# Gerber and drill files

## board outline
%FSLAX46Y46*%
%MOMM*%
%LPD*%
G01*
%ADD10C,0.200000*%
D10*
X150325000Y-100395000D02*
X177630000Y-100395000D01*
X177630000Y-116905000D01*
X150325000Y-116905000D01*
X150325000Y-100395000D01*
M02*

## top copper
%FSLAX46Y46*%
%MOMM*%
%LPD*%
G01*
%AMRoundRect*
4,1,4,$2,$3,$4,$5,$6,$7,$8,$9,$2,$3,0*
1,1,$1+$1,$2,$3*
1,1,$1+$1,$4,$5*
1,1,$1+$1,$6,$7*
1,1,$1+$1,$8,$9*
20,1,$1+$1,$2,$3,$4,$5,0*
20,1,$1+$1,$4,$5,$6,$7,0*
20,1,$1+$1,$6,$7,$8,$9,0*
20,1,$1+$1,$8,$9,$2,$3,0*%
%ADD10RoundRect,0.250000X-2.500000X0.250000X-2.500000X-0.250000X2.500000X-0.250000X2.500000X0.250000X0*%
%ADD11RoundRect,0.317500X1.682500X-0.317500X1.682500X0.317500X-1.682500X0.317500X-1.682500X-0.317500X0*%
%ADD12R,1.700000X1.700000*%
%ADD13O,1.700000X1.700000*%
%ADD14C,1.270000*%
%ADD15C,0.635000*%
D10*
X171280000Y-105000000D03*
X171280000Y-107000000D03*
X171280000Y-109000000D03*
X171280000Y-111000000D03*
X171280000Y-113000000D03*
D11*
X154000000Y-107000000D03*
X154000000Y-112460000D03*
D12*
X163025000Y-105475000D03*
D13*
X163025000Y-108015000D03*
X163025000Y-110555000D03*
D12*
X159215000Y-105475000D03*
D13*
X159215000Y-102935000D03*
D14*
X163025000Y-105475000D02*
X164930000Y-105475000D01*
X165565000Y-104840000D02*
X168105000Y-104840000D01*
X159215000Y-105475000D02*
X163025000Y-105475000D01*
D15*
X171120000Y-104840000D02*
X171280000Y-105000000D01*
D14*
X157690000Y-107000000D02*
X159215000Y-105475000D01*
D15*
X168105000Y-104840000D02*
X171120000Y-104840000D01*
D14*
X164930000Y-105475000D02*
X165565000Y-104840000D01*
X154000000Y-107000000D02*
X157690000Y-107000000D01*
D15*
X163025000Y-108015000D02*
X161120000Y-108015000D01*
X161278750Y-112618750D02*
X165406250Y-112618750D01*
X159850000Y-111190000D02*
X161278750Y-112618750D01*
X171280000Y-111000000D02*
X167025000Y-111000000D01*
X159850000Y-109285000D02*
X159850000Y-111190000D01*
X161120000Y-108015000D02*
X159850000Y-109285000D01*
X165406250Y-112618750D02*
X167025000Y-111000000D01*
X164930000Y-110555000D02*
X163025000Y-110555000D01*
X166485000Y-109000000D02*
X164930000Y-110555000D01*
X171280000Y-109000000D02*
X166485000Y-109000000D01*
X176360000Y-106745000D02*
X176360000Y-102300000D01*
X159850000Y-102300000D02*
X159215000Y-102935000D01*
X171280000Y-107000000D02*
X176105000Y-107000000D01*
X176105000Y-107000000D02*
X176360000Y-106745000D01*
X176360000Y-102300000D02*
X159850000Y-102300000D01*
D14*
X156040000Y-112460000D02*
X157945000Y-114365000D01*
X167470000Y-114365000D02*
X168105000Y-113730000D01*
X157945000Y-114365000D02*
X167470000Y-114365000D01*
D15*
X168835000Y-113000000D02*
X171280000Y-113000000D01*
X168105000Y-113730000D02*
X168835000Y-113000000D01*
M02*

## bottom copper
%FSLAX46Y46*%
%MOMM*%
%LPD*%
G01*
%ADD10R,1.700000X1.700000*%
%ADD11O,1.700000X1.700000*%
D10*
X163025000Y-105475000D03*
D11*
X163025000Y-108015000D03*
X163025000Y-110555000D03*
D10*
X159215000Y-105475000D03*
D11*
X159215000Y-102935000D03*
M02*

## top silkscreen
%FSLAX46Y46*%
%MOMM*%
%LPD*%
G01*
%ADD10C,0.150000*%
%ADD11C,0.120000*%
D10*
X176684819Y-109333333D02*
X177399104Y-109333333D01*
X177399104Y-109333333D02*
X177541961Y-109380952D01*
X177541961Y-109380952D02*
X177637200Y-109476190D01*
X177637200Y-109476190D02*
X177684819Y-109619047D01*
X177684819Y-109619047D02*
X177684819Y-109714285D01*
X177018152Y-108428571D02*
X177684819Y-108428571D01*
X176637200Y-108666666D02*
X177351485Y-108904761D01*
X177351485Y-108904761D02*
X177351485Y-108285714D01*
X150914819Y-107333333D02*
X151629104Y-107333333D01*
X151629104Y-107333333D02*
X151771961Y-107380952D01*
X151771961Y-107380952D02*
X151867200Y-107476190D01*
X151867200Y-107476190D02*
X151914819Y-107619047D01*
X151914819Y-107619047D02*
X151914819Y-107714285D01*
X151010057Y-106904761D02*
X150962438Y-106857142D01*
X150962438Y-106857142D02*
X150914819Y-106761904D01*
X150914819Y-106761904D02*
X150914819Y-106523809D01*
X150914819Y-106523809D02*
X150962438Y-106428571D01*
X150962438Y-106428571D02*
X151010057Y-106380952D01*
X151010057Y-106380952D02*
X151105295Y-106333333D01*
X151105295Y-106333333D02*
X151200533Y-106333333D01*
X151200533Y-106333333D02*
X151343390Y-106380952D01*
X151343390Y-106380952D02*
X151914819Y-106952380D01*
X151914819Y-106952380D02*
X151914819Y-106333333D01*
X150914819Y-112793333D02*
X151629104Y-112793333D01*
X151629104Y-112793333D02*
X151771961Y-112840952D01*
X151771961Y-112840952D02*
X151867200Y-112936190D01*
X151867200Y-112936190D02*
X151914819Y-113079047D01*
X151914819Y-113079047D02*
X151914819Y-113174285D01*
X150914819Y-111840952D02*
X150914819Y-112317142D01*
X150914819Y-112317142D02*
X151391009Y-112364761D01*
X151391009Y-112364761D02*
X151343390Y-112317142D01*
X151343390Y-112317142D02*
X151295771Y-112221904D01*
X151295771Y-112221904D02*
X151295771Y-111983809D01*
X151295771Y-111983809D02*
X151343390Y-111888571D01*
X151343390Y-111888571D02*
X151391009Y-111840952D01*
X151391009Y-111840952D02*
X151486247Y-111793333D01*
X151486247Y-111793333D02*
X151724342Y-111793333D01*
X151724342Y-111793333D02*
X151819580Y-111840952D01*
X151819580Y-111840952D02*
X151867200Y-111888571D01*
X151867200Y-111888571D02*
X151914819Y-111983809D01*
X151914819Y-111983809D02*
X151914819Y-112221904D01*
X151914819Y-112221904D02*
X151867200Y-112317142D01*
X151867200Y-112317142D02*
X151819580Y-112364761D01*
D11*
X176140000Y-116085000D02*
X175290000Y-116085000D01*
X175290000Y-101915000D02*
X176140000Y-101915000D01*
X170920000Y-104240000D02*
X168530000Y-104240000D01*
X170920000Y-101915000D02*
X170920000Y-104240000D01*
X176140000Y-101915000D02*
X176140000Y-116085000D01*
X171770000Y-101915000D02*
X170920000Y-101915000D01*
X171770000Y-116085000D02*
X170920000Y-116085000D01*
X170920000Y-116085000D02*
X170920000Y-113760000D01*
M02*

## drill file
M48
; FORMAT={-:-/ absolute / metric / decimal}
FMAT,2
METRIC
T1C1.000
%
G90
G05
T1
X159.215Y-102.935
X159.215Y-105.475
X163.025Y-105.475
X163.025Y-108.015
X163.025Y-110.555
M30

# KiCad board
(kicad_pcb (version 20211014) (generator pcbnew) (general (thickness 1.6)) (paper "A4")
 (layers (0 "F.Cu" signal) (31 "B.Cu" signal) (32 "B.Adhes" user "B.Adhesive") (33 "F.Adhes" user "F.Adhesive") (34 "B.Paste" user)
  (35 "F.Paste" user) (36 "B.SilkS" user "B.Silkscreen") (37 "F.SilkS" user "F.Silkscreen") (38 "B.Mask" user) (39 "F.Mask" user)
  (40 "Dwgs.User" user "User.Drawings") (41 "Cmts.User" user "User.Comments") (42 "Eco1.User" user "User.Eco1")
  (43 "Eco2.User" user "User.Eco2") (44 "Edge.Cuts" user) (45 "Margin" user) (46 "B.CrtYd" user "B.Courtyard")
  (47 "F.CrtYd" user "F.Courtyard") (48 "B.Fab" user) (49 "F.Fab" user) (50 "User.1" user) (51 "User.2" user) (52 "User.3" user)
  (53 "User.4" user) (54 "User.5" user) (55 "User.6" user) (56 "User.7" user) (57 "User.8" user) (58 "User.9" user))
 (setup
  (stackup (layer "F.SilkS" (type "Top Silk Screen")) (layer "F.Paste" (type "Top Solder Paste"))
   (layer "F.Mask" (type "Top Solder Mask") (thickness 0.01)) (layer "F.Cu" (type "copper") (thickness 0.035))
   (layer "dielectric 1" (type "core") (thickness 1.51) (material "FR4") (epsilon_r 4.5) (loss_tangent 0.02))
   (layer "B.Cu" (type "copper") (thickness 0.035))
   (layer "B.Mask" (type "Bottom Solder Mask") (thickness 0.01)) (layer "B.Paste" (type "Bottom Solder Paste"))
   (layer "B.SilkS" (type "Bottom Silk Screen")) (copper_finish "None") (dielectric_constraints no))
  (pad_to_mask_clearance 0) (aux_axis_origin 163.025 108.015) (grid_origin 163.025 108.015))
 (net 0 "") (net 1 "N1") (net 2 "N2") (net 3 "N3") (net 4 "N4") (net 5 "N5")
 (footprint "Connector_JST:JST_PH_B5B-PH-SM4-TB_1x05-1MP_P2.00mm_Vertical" (layer "F.Cu") (at 171.78 109 -90)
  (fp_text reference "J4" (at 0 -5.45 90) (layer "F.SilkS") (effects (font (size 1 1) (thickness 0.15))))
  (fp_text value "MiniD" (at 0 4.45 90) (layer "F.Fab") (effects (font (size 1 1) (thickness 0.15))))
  (fp_line (start 7.085 -4.36) (end 7.085 -3.51) (layer "F.SilkS") (width 0.12))
  (fp_line (start -7.085 -3.51) (end -7.085 -4.36) (layer "F.SilkS") (width 0.12))
  (fp_line (start -4.76 0.86) (end -4.76 3.25) (layer "F.SilkS") (width 0.12))
  (fp_line (start -7.085 0.86) (end -4.76 0.86) (layer "F.SilkS") (width 0.12))
  (fp_line (start -7.085 -4.36) (end 7.085 -4.36) (layer "F.SilkS") (width 0.12))
  (fp_line (start -7.085 0.01) (end -7.085 0.86) (layer "F.SilkS") (width 0.12))
  (fp_line (start 7.085 0.01) (end 7.085 0.86) (layer "F.SilkS") (width 0.12))
  (fp_line (start 7.085 0.86) (end 4.76 0.86) (layer "F.SilkS") (width 0.12))
  (pad "1" smd roundrect (at -4 0.5 270) (size 1 5.5) (layers "F.Cu" "F.Paste" "F.Mask") (roundrect_rratio 0.25) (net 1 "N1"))
  (pad "2" smd roundrect (at -2 0.5 270) (size 1 5.5) (layers "F.Cu" "F.Paste" "F.Mask") (roundrect_rratio 0.25) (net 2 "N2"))
  (pad "3" smd roundrect (at 0 0.5 270) (size 1 5.5) (layers "F.Cu" "F.Paste" "F.Mask") (roundrect_rratio 0.25) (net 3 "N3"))
  (pad "4" smd roundrect (at 2 0.5 270) (size 1 5.5) (layers "F.Cu" "F.Paste" "F.Mask") (roundrect_rratio 0.25) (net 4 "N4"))
  (pad "5" smd roundrect (at 4 0.5 270) (size 1 5.5) (layers "F.Cu" "F.Paste" "F.Mask") (roundrect_rratio 0.25) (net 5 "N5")))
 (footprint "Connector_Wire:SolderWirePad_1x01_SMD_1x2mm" (layer "F.Cu") (at 154 107 90)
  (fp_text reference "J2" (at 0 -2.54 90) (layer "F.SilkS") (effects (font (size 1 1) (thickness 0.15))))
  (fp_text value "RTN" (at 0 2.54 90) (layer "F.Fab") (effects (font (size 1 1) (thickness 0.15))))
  (pad "1" smd roundrect (at 0 0 90) (size 1.27 4) (layers "F.Cu" "F.Paste" "F.Mask") (roundrect_rratio 0.25) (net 1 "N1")))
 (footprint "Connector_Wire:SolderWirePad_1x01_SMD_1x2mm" (layer "F.Cu") (at 154 112.46 90)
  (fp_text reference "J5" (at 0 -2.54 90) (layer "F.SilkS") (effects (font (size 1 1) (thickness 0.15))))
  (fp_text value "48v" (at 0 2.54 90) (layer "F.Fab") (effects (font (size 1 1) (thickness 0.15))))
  (pad "1" smd roundrect (at 0 0 90) (size 1.27 4) (layers "F.Cu" "F.Paste" "F.Mask") (roundrect_rratio 0.25) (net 5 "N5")))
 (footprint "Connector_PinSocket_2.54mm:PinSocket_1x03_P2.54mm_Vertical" (layer "B.Cu") (at 163.025 105.475 180)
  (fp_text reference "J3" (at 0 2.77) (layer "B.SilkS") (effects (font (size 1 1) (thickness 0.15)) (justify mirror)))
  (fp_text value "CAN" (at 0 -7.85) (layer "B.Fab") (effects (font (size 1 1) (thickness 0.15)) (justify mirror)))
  (pad "1" thru_hole rect (at 0 0 180) (size 1.7 1.7) (drill 1) (layers *.Cu *.Mask) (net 1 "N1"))
  (pad "2" thru_hole oval (at 0 -2.54 180) (size 1.7 1.7) (drill 1) (layers *.Cu *.Mask) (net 4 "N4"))
  (pad "3" thru_hole oval (at 0 -5.08 180) (size 1.7 1.7) (drill 1) (layers *.Cu *.Mask) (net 3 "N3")))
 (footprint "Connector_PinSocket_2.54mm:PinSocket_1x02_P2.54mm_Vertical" (layer "B.Cu") (at 159.215 105.475)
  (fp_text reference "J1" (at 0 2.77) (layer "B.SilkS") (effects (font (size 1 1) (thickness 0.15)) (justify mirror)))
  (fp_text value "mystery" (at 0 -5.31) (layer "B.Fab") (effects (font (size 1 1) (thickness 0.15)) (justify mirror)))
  (pad "1" thru_hole rect (at 0 0) (size 1.7 1.7) (drill 1) (layers *.Cu *.Mask) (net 1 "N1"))
  (pad "2" thru_hole oval (at 0 -2.54) (size 1.7 1.7) (drill 1) (layers *.Cu *.Mask) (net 2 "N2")))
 (gr_rect (start 150.325 100.395) (end 177.63 116.905) (layer "Edge.Cuts") (width 0.2) (fill none))
 (segment (start 163.025 105.475) (end 164.93 105.475) (width 1.27) (layer "F.Cu") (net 1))
 (segment (start 165.565 104.84) (end 168.105 104.84) (width 1.27) (layer "F.Cu") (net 1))
 (segment (start 159.215 105.475) (end 163.025 105.475) (width 1.27) (layer "F.Cu") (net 1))
 (segment (start 171.12 104.84) (end 171.28 105) (width 0.635) (layer "F.Cu") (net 1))
 (segment (start 157.69 107) (end 159.215 105.475) (width 1.27) (layer "F.Cu") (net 1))
 (segment (start 168.105 104.84) (end 171.12 104.84) (width 0.635) (layer "F.Cu") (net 1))
 (segment (start 164.93 105.475) (end 165.565 104.84) (width 1.27) (layer "F.Cu") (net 1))
 (segment (start 154 107) (end 157.69 107) (width 1.27) (layer "F.Cu") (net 1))
 (segment (start 163.025 108.015) (end 161.12 108.015) (width 0.635) (layer "F.Cu") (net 4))
 (segment (start 161.27875 112.61875) (end 165.40625 112.61875) (width 0.635) (layer "F.Cu") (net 4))
 (segment (start 159.85 111.19) (end 161.27875 112.61875) (width 0.635) (layer "F.Cu") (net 4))
 (segment (start 171.28 111) (end 167.025 111) (width 0.635) (layer "F.Cu") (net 4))
 (segment (start 159.85 109.285) (end 159.85 111.19) (width 0.635) (layer "F.Cu") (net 4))
 (segment (start 161.12 108.015) (end 159.85 109.285) (width 0.635) (layer "F.Cu") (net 4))
 (segment (start 165.40625 112.61875) (end 167.025 111) (width 0.635) (layer "F.Cu") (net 4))
 (segment (start 164.93 110.555) (end 163.025 110.555) (width 0.635) (layer "F.Cu") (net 3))
 (segment (start 166.485 109) (end 164.93 110.555) (width 0.635) (layer "F.Cu") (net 3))
 (segment (start 171.28 109) (end 166.485 109) (width 0.635) (layer "F.Cu") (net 3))
 (segment (start 176.36 106.745) (end 176.36 102.3) (width 0.635) (layer "F.Cu") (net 2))
 (segment (start 159.85 102.3) (end 159.215 102.935) (width 0.635) (layer "F.Cu") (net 2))
 (segment (start 171.28 107) (end 176.105 107) (width 0.635) (layer "F.Cu") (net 2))
 (segment (start 176.105 107) (end 176.36 106.745) (width 0.635) (layer "F.Cu") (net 2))
 (segment (start 176.36 102.3) (end 159.85 102.3) (width 0.635) (layer "F.Cu") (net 2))
 (segment (start 156.04 112.46) (end 157.945 114.365) (width 1.27) (layer "F.Cu") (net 5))
 (segment (start 167.47 114.365) (end 168.105 113.73) (width 1.27) (layer "F.Cu") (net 5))
 (segment (start 157.945 114.365) (end 167.47 114.365) (width 1.27) (layer "F.Cu") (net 5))
 (segment (start 168.835 113) (end 171.28 113) (width 0.635) (layer "F.Cu") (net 5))
 (segment (start 168.105 113.73) (end 168.835 113) (width 0.635) (layer "F.Cu") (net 5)))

